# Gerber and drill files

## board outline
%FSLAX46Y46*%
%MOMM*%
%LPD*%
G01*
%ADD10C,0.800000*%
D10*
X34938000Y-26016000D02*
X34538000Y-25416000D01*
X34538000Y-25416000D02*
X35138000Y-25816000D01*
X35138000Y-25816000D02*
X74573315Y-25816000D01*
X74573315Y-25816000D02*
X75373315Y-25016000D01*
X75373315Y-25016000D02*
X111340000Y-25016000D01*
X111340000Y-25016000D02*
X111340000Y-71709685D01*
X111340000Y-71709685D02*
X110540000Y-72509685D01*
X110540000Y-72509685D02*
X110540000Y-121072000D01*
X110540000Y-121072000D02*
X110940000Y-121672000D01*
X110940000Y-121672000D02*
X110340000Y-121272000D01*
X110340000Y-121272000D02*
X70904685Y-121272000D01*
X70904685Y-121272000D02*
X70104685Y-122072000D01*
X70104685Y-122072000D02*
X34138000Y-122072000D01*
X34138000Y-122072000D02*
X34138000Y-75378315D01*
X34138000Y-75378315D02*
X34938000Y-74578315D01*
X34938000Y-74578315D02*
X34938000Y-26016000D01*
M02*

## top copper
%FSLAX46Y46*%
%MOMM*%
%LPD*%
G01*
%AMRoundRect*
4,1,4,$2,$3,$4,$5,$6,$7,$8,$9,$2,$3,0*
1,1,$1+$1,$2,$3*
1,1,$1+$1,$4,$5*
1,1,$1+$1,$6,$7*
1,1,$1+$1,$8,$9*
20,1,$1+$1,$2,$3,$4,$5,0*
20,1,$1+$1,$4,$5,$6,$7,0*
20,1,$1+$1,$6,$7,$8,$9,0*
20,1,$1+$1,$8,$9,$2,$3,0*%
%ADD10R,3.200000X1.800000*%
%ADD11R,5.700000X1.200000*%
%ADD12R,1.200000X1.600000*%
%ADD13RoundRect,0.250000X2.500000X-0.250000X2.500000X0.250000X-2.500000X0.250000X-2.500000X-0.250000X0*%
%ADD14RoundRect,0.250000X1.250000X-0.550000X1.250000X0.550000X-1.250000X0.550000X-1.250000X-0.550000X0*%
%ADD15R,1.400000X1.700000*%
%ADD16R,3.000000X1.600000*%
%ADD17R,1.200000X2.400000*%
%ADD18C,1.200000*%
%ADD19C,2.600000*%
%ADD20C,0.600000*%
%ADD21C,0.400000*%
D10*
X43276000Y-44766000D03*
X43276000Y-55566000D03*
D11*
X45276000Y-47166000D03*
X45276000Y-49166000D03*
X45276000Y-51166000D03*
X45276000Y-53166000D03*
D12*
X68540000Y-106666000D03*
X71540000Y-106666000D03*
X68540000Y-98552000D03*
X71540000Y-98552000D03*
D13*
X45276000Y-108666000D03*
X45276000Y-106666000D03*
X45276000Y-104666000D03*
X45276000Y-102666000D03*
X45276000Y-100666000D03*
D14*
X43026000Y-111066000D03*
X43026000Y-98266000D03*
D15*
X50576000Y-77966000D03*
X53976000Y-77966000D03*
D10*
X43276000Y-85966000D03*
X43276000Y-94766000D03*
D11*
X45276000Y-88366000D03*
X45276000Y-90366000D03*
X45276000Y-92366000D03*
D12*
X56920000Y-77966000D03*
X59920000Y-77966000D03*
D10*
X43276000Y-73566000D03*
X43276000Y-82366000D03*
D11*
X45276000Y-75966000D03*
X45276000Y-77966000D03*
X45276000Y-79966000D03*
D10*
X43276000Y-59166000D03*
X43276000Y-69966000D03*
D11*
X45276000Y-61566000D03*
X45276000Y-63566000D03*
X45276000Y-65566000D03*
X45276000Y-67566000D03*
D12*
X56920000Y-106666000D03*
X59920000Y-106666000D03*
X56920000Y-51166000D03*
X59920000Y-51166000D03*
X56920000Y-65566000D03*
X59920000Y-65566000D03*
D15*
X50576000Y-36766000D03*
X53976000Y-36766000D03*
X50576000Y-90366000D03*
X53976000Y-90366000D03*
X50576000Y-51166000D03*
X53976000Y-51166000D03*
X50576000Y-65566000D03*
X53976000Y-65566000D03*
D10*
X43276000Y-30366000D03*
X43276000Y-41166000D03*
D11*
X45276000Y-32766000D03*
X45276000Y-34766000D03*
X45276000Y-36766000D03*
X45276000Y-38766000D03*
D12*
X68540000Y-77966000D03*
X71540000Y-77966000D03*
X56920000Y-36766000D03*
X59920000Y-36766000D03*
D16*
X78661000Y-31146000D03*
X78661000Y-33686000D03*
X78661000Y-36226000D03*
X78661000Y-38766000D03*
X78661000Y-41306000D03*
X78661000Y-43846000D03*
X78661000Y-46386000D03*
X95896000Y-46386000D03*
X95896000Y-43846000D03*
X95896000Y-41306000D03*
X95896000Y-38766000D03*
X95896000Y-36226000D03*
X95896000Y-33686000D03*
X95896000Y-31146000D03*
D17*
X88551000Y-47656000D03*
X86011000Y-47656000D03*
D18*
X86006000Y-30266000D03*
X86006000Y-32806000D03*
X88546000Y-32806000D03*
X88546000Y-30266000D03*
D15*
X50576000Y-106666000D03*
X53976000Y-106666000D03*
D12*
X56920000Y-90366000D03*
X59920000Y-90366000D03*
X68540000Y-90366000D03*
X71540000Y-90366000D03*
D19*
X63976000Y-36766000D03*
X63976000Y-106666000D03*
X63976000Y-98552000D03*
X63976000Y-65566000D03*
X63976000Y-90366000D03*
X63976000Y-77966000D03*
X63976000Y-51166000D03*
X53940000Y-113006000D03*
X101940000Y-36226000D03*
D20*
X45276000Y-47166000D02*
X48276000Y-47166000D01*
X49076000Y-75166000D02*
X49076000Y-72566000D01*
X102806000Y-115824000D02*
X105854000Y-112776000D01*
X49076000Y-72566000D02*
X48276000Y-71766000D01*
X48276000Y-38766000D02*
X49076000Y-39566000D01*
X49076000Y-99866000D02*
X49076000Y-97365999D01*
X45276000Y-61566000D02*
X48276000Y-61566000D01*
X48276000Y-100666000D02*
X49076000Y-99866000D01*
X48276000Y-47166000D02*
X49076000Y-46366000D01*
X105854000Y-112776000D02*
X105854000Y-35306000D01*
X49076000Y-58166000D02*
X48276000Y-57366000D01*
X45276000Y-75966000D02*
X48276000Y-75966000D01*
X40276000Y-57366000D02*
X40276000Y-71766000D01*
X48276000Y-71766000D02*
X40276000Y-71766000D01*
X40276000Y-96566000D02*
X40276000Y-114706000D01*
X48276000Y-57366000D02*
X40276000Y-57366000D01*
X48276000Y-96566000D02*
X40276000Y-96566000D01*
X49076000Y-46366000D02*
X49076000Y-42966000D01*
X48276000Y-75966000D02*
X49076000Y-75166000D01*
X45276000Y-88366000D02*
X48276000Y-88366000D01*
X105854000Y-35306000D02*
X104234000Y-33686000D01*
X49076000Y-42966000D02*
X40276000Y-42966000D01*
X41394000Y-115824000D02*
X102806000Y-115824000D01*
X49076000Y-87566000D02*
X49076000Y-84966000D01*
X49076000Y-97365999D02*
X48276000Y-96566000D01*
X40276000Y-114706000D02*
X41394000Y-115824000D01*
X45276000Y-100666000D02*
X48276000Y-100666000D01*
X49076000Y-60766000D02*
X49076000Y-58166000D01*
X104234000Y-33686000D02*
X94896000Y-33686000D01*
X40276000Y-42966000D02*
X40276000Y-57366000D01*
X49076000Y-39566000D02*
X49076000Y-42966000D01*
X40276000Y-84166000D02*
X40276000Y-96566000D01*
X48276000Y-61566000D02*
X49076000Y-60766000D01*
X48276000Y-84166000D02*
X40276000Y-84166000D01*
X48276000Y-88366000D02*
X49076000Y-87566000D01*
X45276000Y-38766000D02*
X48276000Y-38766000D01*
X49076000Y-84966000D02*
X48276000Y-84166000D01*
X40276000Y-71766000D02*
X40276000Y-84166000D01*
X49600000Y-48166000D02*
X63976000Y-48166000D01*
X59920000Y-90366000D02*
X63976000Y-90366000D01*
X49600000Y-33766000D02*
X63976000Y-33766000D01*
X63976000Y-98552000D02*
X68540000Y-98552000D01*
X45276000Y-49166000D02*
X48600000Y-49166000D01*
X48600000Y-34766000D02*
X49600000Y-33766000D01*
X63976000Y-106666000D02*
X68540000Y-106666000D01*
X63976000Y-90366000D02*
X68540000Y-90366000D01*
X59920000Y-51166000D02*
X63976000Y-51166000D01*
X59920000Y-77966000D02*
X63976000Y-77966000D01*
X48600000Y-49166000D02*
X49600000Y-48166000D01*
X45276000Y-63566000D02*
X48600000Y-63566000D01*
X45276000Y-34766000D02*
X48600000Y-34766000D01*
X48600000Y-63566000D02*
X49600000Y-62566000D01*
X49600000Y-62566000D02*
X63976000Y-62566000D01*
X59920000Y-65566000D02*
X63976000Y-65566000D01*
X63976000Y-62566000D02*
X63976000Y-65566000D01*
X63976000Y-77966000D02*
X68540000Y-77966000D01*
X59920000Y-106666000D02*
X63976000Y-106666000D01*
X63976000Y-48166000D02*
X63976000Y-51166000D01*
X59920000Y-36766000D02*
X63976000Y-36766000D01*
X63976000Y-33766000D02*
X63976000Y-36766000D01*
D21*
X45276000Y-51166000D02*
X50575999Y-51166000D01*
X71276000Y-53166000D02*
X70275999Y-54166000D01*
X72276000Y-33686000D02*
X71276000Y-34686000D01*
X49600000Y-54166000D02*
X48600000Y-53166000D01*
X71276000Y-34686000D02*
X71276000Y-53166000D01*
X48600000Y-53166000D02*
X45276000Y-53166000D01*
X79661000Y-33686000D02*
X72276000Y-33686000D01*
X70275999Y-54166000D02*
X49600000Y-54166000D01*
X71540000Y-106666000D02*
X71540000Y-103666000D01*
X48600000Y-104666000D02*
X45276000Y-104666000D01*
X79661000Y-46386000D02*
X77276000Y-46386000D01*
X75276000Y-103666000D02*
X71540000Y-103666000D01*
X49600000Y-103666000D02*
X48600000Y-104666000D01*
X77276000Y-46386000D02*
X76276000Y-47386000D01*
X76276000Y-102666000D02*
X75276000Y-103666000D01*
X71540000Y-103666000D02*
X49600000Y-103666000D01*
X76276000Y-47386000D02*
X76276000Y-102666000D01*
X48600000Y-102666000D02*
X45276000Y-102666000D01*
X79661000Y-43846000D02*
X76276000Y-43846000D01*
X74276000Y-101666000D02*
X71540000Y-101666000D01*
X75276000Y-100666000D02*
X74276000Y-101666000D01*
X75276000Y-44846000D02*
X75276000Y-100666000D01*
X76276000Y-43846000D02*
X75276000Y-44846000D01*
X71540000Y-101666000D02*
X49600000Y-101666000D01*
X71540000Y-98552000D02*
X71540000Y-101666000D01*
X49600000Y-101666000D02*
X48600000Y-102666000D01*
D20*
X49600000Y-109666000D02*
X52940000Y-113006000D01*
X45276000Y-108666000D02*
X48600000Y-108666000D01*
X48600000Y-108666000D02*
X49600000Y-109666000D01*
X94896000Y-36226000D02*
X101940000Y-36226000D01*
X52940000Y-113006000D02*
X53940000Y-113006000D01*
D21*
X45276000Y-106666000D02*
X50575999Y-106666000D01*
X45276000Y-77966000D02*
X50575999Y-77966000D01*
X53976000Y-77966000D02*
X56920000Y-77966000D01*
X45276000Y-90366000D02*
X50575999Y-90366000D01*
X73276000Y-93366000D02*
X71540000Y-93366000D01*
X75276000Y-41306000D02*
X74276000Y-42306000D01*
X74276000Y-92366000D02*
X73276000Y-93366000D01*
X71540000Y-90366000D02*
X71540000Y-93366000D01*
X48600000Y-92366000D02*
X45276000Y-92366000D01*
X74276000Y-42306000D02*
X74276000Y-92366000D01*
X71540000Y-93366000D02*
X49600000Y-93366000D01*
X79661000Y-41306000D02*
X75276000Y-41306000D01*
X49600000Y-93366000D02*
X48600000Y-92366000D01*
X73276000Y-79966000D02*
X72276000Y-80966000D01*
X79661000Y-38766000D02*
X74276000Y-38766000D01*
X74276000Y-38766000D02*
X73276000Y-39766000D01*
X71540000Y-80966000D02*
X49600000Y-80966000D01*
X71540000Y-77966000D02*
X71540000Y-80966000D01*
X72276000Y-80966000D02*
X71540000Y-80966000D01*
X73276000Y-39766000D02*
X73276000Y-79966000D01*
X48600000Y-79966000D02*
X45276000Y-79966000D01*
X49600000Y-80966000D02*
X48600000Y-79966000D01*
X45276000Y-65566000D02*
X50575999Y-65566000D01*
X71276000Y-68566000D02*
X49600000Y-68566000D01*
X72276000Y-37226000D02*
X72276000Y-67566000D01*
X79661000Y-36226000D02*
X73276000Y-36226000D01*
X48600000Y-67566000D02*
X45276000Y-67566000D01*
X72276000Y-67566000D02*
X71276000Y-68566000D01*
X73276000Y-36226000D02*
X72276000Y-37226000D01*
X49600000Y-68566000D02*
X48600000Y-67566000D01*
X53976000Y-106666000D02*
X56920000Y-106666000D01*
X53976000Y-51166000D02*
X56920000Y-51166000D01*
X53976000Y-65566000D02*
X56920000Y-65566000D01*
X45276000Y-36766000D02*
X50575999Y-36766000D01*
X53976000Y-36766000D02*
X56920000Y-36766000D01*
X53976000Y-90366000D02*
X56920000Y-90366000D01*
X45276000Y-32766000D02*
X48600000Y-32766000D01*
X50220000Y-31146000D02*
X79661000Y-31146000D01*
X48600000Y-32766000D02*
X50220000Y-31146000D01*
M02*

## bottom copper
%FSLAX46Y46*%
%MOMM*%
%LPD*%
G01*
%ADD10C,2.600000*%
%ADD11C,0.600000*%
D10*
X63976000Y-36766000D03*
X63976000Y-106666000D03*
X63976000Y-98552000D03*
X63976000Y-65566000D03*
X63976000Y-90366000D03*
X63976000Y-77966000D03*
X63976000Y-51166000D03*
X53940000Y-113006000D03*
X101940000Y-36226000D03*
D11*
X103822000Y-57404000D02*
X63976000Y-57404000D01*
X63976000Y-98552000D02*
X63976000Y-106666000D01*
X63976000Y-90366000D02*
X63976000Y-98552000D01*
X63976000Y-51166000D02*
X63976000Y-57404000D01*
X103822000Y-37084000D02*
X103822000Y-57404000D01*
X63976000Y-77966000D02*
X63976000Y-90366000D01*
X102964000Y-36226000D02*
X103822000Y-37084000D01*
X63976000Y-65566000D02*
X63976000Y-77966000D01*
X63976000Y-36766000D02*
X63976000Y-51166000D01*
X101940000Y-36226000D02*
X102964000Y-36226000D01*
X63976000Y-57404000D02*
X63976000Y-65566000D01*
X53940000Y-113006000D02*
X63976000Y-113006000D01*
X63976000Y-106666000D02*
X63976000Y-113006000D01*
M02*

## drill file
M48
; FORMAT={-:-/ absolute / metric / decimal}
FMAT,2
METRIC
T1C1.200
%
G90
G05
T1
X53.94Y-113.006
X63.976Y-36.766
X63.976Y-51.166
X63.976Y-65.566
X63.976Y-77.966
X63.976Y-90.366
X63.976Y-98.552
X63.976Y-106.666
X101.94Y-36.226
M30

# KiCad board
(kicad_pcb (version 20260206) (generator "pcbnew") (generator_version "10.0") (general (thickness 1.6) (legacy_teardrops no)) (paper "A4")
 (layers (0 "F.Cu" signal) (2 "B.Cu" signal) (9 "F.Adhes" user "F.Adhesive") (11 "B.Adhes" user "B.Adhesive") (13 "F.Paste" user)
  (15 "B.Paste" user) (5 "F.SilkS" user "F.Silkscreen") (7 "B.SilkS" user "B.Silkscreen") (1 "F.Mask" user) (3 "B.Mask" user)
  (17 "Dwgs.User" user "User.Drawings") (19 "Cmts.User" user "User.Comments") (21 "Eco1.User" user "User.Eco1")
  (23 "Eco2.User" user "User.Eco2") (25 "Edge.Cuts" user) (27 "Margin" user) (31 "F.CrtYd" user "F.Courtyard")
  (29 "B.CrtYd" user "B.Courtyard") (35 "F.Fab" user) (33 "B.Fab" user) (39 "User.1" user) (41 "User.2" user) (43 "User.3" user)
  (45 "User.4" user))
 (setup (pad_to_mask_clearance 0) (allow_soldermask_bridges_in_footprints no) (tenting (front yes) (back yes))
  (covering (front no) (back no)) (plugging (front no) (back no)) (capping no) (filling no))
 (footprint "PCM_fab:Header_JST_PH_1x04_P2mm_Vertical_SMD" (layer "F.Cu") (at 45.276 48.166)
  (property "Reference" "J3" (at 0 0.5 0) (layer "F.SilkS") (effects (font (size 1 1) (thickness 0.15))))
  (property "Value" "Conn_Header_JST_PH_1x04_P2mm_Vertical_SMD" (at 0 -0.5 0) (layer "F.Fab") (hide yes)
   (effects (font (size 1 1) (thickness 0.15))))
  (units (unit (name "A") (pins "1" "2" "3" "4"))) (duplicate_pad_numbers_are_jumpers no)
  (pad "" smd rect (at -2 -3.4) (size 3.2 1.8) (layers "F.Cu" "F.Mask" "F.Paste"))
  (pad "" smd rect (at -2 7.4) (size 3.2 1.8) (layers "F.Cu" "F.Mask" "F.Paste"))
  (pad "1" smd rect (at 0 -1) (size 5.7 1.2) (layers "F.Cu" "F.Mask" "F.Paste") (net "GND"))
  (pad "2" smd rect (at 0 1) (size 5.7 1.2) (layers "F.Cu" "F.Mask" "F.Paste") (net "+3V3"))
  (pad "3" smd rect (at 0 3) (size 5.7 1.2) (layers "F.Cu" "F.Mask" "F.Paste") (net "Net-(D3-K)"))
  (pad "4" smd rect (at 0 5) (size 5.7 1.2) (layers "F.Cu" "F.Mask" "F.Paste") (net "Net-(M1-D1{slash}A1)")))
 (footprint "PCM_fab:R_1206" (layer "F.Cu") (at 70.04 106.666)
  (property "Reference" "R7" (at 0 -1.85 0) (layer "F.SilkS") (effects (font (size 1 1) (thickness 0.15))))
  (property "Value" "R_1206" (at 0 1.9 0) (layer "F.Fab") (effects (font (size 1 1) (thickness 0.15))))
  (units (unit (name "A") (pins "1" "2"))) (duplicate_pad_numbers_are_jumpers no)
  (pad "1" smd rect (at -1.5 0) (size 1.2 1.6) (layers "F.Cu" "F.Mask" "F.Paste") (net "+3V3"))
  (pad "2" smd rect (at 1.5 0) (size 1.2 1.6) (layers "F.Cu" "F.Mask" "F.Paste") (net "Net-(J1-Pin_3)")))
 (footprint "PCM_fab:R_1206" (layer "F.Cu") (at 70.04 98.552)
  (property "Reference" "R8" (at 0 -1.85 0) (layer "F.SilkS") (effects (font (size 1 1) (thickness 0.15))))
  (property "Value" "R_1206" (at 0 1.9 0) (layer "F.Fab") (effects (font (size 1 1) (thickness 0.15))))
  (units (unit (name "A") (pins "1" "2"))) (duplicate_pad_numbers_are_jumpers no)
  (pad "1" smd rect (at -1.5 0) (size 1.2 1.6) (layers "F.Cu" "F.Mask" "F.Paste") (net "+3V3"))
  (pad "2" smd rect (at 1.5 0) (size 1.2 1.6) (layers "F.Cu" "F.Mask" "F.Paste") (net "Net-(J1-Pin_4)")))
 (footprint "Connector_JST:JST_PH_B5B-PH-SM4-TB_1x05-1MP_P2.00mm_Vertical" (layer "F.Cu") (at 44.776 104.666 90)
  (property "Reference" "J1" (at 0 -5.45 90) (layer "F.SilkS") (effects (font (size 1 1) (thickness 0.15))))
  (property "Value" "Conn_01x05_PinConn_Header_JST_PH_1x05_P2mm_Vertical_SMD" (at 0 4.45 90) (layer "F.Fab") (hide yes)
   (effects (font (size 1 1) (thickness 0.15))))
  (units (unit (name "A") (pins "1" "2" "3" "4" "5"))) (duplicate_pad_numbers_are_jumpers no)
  (pad "1" smd roundrect (at -4 0.5 90) (size 1 5.5) (layers "F.Cu" "F.Mask" "F.Paste") (roundrect_rratio 0.25) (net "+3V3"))
  (pad "2" smd roundrect (at -2 0.5 90) (size 1 5.5) (layers "F.Cu" "F.Mask" "F.Paste") (roundrect_rratio 0.25) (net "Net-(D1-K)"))
  (pad "3" smd roundrect (at 0 0.5 90) (size 1 5.5) (layers "F.Cu" "F.Mask" "F.Paste") (roundrect_rratio 0.25) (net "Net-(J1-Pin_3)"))
  (pad "4" smd roundrect (at 2 0.5 90) (size 1 5.5) (layers "F.Cu" "F.Mask" "F.Paste") (roundrect_rratio 0.25) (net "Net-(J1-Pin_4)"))
  (pad "5" smd roundrect (at 4 0.5 90) (size 1 5.5) (layers "F.Cu" "F.Mask" "F.Paste") (roundrect_rratio 0.25) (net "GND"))
  (pad "MP" smd roundrect (at -6.4 -1.75 90) (size 1.6 3) (layers "F.Cu" "F.Mask" "F.Paste") (roundrect_rratio 0.15625))
  (pad "MP" smd roundrect (at 6.4 -1.75 90) (size 1.6 3) (layers "F.Cu" "F.Mask" "F.Paste") (roundrect_rratio 0.15625)))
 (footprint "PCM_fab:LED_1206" (layer "F.Cu") (at 52.276 77.966)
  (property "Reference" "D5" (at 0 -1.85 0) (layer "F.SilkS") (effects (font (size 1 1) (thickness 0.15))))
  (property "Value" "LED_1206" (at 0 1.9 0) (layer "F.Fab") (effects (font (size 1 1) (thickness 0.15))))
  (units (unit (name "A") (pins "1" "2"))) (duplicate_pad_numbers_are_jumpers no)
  (pad "1" smd rect (at -1.7 0) (size 1.4 1.7) (layers "F.Cu" "F.Mask" "F.Paste") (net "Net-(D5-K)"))
  (pad "2" smd rect (at 1.7 0) (size 1.4 1.7) (layers "F.Cu" "F.Mask" "F.Paste") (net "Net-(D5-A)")))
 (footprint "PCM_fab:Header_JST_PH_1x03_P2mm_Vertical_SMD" (layer "F.Cu") (at 45.276 89.366)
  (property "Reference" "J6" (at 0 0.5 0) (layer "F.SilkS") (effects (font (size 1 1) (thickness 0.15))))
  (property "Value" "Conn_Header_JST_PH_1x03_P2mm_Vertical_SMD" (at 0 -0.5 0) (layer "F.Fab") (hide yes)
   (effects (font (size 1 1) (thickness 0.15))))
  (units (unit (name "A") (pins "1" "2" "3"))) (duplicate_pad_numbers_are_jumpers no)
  (pad "" smd rect (at -2 -3.4) (size 3.2 1.8) (layers "F.Cu" "F.Mask" "F.Paste"))
  (pad "" smd rect (at -2 5.4) (size 3.2 1.8) (layers "F.Cu" "F.Mask" "F.Paste"))
  (pad "1" smd rect (at 0 -1) (size 5.7 1.2) (layers "F.Cu" "F.Mask" "F.Paste") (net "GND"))
  (pad "2" smd rect (at 0 1) (size 5.7 1.2) (layers "F.Cu" "F.Mask" "F.Paste") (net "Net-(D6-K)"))
  (pad "3" smd rect (at 0 3) (size 5.7 1.2) (layers "F.Cu" "F.Mask" "F.Paste") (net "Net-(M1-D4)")))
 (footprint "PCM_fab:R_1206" (layer "F.Cu") (at 58.42 77.966)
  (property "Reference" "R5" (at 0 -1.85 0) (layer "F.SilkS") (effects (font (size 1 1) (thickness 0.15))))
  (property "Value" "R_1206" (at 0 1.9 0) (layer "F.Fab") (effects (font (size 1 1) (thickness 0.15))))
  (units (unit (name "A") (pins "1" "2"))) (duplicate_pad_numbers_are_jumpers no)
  (pad "1" smd rect (at -1.5 0) (size 1.2 1.6) (layers "F.Cu" "F.Mask" "F.Paste") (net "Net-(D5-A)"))
  (pad "2" smd rect (at 1.5 0) (size 1.2 1.6) (layers "F.Cu" "F.Mask" "F.Paste") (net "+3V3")))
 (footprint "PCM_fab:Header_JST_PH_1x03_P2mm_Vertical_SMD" (layer "F.Cu") (at 45.276 76.966)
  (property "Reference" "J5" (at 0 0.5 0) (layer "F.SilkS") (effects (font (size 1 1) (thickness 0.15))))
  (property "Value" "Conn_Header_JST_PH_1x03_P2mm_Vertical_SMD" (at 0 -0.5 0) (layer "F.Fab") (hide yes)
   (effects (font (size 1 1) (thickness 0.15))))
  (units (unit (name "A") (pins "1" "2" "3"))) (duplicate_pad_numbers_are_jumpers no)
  (pad "" smd rect (at -2 -3.4) (size 3.2 1.8) (layers "F.Cu" "F.Mask" "F.Paste"))
  (pad "" smd rect (at -2 5.4) (size 3.2 1.8) (layers "F.Cu" "F.Mask" "F.Paste"))
  (pad "1" smd rect (at 0 -1) (size 5.7 1.2) (layers "F.Cu" "F.Mask" "F.Paste") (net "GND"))
  (pad "2" smd rect (at 0 1) (size 5.7 1.2) (layers "F.Cu" "F.Mask" "F.Paste") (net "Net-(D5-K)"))
  (pad "3" smd rect (at 0 3) (size 5.7 1.2) (layers "F.Cu" "F.Mask" "F.Paste") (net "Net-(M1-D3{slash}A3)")))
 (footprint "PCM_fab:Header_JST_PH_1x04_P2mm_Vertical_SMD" (layer "F.Cu") (at 45.276 62.566)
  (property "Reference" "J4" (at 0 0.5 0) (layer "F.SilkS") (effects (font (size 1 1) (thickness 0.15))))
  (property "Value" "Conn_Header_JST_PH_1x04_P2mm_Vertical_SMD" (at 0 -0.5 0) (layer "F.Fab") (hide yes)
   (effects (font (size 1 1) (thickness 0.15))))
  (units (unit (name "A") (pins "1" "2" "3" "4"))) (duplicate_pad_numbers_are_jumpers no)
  (pad "" smd rect (at -2 -3.4) (size 3.2 1.8) (layers "F.Cu" "F.Mask" "F.Paste"))
  (pad "" smd rect (at -2 7.4) (size 3.2 1.8) (layers "F.Cu" "F.Mask" "F.Paste"))
  (pad "1" smd rect (at 0 -1) (size 5.7 1.2) (layers "F.Cu" "F.Mask" "F.Paste") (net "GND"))
  (pad "2" smd rect (at 0 1) (size 5.7 1.2) (layers "F.Cu" "F.Mask" "F.Paste") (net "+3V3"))
  (pad "3" smd rect (at 0 3) (size 5.7 1.2) (layers "F.Cu" "F.Mask" "F.Paste") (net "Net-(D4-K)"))
  (pad "4" smd rect (at 0 5) (size 5.7 1.2) (layers "F.Cu" "F.Mask" "F.Paste") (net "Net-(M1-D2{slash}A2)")))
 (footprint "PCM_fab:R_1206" (layer "F.Cu") (at 58.42 106.666)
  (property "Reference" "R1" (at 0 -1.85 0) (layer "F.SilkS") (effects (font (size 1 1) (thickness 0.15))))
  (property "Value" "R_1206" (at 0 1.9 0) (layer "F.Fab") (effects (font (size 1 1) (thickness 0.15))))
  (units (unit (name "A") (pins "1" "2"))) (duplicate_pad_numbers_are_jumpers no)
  (pad "1" smd rect (at -1.5 0) (size 1.2 1.6) (layers "F.Cu" "F.Mask" "F.Paste") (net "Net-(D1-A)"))
  (pad "2" smd rect (at 1.5 0) (size 1.2 1.6) (layers "F.Cu" "F.Mask" "F.Paste") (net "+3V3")))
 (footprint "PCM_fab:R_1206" (layer "F.Cu") (at 58.42 51.166)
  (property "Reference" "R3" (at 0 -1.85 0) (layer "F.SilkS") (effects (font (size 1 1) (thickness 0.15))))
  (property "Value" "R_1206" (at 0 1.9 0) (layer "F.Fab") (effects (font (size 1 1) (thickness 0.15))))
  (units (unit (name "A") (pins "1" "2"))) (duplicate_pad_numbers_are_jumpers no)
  (pad "1" smd rect (at -1.5 0) (size 1.2 1.6) (layers "F.Cu" "F.Mask" "F.Paste") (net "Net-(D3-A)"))
  (pad "2" smd rect (at 1.5 0) (size 1.2 1.6) (layers "F.Cu" "F.Mask" "F.Paste") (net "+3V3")))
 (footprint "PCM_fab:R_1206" (layer "F.Cu") (at 58.42 65.566)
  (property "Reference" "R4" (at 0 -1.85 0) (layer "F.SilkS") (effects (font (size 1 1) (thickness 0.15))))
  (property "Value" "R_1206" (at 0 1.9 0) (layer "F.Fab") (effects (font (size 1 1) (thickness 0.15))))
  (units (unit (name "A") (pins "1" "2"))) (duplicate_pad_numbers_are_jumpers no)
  (pad "1" smd rect (at -1.5 0) (size 1.2 1.6) (layers "F.Cu" "F.Mask" "F.Paste") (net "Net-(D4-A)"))
  (pad "2" smd rect (at 1.5 0) (size 1.2 1.6) (layers "F.Cu" "F.Mask" "F.Paste") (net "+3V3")))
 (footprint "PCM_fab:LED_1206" (layer "F.Cu") (at 52.276 36.766)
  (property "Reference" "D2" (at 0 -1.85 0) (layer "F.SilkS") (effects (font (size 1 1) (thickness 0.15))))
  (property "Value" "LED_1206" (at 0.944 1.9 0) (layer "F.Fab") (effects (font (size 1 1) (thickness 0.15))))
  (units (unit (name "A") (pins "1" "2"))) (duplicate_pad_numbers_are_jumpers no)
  (pad "1" smd rect (at -1.7 0) (size 1.4 1.7) (layers "F.Cu" "F.Mask" "F.Paste") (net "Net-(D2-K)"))
  (pad "2" smd rect (at 1.7 0) (size 1.4 1.7) (layers "F.Cu" "F.Mask" "F.Paste") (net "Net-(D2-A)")))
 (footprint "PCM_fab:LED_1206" (layer "F.Cu") (at 52.276 90.366)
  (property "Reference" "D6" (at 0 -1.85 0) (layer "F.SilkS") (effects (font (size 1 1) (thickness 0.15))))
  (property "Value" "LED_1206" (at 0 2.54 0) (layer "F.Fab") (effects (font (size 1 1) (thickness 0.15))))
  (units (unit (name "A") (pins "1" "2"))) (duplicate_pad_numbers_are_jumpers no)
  (pad "1" smd rect (at -1.7 0) (size 1.4 1.7) (layers "F.Cu" "F.Mask" "F.Paste") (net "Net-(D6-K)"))
  (pad "2" smd rect (at 1.7 0) (size 1.4 1.7) (layers "F.Cu" "F.Mask" "F.Paste") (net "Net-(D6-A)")))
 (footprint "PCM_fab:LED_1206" (layer "F.Cu") (at 52.276 51.166)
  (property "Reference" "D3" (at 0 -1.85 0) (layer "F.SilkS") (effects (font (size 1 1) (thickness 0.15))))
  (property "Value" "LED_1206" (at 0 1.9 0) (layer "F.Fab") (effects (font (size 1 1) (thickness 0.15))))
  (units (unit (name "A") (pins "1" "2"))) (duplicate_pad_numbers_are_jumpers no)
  (pad "1" smd rect (at -1.7 0) (size 1.4 1.7) (layers "F.Cu" "F.Mask" "F.Paste") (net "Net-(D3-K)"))
  (pad "2" smd rect (at 1.7 0) (size 1.4 1.7) (layers "F.Cu" "F.Mask" "F.Paste") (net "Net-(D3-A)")))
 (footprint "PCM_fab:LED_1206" (layer "F.Cu") (at 52.276 65.566)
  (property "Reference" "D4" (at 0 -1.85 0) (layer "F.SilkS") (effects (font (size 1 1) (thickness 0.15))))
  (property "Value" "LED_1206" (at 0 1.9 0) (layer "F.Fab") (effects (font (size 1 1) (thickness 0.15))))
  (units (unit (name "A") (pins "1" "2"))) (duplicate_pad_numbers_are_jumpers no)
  (pad "1" smd rect (at -1.7 0) (size 1.4 1.7) (layers "F.Cu" "F.Mask" "F.Paste") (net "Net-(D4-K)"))
  (pad "2" smd rect (at 1.7 0) (size 1.4 1.7) (layers "F.Cu" "F.Mask" "F.Paste") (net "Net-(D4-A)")))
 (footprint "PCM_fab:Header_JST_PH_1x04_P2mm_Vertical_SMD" (layer "F.Cu") (at 45.276 33.766)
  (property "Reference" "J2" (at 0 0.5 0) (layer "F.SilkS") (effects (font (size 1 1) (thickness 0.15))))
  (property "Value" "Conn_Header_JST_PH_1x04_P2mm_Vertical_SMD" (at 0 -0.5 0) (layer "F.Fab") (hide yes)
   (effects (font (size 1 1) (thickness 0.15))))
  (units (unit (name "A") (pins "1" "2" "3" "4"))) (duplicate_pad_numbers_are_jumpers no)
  (pad "" smd rect (at -2 -3.4) (size 3.2 1.8) (layers "F.Cu" "F.Mask" "F.Paste"))
  (pad "" smd rect (at -2 7.4) (size 3.2 1.8) (layers "F.Cu" "F.Mask" "F.Paste"))
  (pad "1" smd rect (at 0 -1) (size 5.7 1.2) (layers "F.Cu" "F.Mask" "F.Paste") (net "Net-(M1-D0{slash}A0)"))
  (pad "2" smd rect (at 0 1) (size 5.7 1.2) (layers "F.Cu" "F.Mask" "F.Paste") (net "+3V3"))
  (pad "3" smd rect (at 0 3) (size 5.7 1.2) (layers "F.Cu" "F.Mask" "F.Paste") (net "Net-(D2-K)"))
  (pad "4" smd rect (at 0 5) (size 5.7 1.2) (layers "F.Cu" "F.Mask" "F.Paste") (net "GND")))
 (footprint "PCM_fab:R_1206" (layer "F.Cu") (at 70.04 77.966)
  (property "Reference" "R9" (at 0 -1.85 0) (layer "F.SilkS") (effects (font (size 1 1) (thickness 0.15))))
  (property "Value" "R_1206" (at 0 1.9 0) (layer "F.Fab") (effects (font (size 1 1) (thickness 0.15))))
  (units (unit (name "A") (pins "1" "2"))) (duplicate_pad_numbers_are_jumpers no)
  (pad "1" smd rect (at -1.5 0) (size 1.2 1.6) (layers "F.Cu" "F.Mask" "F.Paste") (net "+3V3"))
  (pad "2" smd rect (at 1.5 0) (size 1.2 1.6) (layers "F.Cu" "F.Mask" "F.Paste") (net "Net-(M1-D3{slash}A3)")))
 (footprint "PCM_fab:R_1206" (layer "F.Cu") (at 58.42 36.766)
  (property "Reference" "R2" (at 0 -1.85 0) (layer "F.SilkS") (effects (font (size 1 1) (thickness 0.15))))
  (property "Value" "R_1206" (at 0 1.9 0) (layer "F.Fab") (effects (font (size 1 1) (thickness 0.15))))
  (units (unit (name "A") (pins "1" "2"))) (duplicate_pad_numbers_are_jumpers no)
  (pad "1" smd rect (at -1.5 0) (size 1.2 1.6) (layers "F.Cu" "F.Mask" "F.Paste") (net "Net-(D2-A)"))
  (pad "2" smd rect (at 1.5 0) (size 1.2 1.6) (layers "F.Cu" "F.Mask" "F.Paste") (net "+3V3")))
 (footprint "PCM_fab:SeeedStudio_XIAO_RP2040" (layer "F.Cu") (at 87.276 38.766)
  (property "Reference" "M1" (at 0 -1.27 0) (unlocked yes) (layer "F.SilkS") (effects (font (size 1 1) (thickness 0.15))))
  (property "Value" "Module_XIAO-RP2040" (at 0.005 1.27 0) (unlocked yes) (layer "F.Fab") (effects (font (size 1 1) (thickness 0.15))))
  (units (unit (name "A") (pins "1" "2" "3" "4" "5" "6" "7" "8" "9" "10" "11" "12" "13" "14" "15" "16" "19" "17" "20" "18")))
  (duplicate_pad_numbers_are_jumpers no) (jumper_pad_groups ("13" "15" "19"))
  (pad "1" smd rect (at -7.615 -7.62) (size 3 1.6) (drill (offset -1 0)) (layers "F.Cu" "F.Mask" "F.Paste") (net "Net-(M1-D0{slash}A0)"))
  (pad "2" smd rect (at -7.615 -5.08) (size 3 1.6) (drill (offset -1 0)) (layers "F.Cu" "F.Mask" "F.Paste") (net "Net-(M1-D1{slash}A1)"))
  (pad "3" smd rect (at -7.615 -2.54) (size 3 1.6) (drill (offset -1 0)) (layers "F.Cu" "F.Mask" "F.Paste") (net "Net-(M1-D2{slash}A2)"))
  (pad "4" smd rect (at -7.615 0) (size 3 1.6) (drill (offset -1 0)) (layers "F.Cu" "F.Mask" "F.Paste") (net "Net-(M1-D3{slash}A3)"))
  (pad "5" smd rect (at -7.615 2.54) (size 3 1.6) (drill (offset -1 0)) (layers "F.Cu" "F.Mask" "F.Paste") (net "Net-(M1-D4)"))
  (pad "6" smd rect (at -7.615 5.08) (size 3 1.6) (drill (offset -1 0)) (layers "F.Cu" "F.Mask" "F.Paste") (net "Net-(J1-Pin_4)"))
  (pad "7" smd rect (at -7.615 7.62) (size 3 1.6) (drill (offset -1 0)) (layers "F.Cu" "F.Mask" "F.Paste") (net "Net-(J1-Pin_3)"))
  (pad "8" smd rect (at 7.62 7.62) (size 3 1.6) (drill (offset 1 0)) (layers "F.Cu" "F.Mask" "F.Paste") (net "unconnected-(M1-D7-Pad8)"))
  (pad "9" smd rect (at 7.62 5.08) (size 3 1.6) (drill (offset 1 0)) (layers "F.Cu" "F.Mask" "F.Paste") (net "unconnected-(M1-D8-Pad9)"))
  (pad "10" smd rect (at 7.62 2.54) (size 3 1.6) (drill (offset 1 0)) (layers "F.Cu" "F.Mask" "F.Paste") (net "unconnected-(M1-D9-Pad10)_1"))
  (pad "11" smd rect (at 7.62 0) (size 3 1.6) (drill (offset 1 0)) (layers "F.Cu" "F.Mask" "F.Paste") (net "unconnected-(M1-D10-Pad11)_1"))
  (pad "12" smd rect (at 7.62 -2.54) (size 3 1.6) (drill (offset 1 0)) (layers "F.Cu" "F.Mask" "F.Paste") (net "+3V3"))
  (pad "13" smd rect (at 7.62 -5.08) (size 3 1.6) (drill (offset 1 0)) (layers "F.Cu" "F.Mask" "F.Paste") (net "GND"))
  (pad "14" smd rect (at 7.62 -7.62) (size 3 1.6) (drill (offset 1 0)) (layers "F.Cu" "F.Mask" "F.Paste") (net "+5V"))
  (pad "15" smd rect (at 1.275 8.89 270) (size 2.4 1.2) (layers "F.Cu" "F.Mask" "F.Paste") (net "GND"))
  (pad "16" smd rect (at -1.265 8.89 270) (size 2.4 1.2) (layers "F.Cu" "F.Mask" "F.Paste") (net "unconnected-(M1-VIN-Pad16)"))
  (pad "17" smd circle (at -1.27 -8.5) (size 1.2 1.2) (layers "F.Cu" "F.Mask" "F.Paste") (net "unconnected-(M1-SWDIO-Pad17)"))
  (pad "18" smd circle (at -1.27 -5.96) (size 1.2 1.2) (layers "F.Cu" "F.Mask" "F.Paste") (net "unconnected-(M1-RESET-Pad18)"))
  (pad "19" smd circle (at 1.27 -5.96) (size 1.2 1.2) (layers "F.Cu" "F.Mask" "F.Paste") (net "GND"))
  (pad "20" smd circle (at 1.27 -8.5) (size 1.2 1.2) (layers "F.Cu" "F.Mask" "F.Paste") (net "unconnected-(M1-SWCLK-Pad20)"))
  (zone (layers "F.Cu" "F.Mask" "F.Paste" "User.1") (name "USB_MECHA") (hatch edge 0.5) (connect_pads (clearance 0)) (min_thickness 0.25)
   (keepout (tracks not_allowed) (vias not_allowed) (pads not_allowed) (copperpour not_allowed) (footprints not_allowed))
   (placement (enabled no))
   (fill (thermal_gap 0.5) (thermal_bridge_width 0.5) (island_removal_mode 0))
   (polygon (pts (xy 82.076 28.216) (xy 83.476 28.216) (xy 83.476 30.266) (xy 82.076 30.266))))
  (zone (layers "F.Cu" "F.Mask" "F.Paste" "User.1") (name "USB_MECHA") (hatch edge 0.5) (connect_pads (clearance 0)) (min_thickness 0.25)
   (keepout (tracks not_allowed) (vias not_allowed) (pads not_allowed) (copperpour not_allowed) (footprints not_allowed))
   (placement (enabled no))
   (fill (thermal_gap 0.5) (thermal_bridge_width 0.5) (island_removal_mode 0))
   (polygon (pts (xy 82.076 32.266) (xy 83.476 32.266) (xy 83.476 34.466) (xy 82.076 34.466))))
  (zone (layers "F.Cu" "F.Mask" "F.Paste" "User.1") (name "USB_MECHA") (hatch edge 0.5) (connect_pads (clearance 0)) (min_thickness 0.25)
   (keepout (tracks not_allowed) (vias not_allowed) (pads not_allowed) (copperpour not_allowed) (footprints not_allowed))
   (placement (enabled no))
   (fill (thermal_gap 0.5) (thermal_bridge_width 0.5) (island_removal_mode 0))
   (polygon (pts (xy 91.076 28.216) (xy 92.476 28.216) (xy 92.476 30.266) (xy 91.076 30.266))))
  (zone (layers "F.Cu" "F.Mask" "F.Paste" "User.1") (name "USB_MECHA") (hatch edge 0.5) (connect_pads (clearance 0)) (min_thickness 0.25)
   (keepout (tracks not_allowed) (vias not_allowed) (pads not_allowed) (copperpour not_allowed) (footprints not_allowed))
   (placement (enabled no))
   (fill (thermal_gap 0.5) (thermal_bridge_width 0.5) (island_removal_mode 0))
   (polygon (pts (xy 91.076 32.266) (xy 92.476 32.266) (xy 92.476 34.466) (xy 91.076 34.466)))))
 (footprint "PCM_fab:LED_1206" (layer "F.Cu") (at 52.276 106.666)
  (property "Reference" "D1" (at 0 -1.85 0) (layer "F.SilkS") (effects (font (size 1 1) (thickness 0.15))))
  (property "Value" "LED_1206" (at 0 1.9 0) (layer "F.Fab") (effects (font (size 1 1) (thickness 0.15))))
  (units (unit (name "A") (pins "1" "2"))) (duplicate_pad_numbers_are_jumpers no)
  (pad "1" smd rect (at -1.7 0) (size 1.4 1.7) (layers "F.Cu" "F.Mask" "F.Paste") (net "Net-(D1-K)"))
  (pad "2" smd rect (at 1.7 0) (size 1.4 1.7) (layers "F.Cu" "F.Mask" "F.Paste") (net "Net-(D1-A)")))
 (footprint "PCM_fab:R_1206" (layer "F.Cu") (at 58.42 90.366)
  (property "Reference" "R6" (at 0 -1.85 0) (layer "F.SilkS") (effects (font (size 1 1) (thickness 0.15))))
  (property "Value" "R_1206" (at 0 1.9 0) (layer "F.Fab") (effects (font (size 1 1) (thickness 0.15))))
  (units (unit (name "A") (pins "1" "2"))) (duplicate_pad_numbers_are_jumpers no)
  (pad "1" smd rect (at -1.5 0) (size 1.2 1.6) (layers "F.Cu" "F.Mask" "F.Paste") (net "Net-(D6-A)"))
  (pad "2" smd rect (at 1.5 0) (size 1.2 1.6) (layers "F.Cu" "F.Mask" "F.Paste") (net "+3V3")))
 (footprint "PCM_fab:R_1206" (layer "F.Cu") (at 70.04 90.366)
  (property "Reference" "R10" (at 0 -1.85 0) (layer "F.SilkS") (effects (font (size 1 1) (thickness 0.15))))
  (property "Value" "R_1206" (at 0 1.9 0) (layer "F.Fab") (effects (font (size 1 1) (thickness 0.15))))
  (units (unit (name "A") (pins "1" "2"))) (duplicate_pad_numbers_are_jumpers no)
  (pad "1" smd rect (at -1.5 0) (size 1.2 1.6) (layers "F.Cu" "F.Mask" "F.Paste") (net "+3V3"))
  (pad "2" smd rect (at 1.5 0) (size 1.2 1.6) (layers "F.Cu" "F.Mask" "F.Paste") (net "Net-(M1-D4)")))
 (gr_line (start 34.938 26.016) (end 34.538 25.416) (stroke (width 0.8) (type solid)) (layer "Edge.Cuts"))
 (gr_line (start 34.538 25.416) (end 35.138 25.816) (stroke (width 0.8) (type solid)) (layer "Edge.Cuts"))
 (gr_line (start 35.138 25.816) (end 74.573315 25.816) (stroke (width 0.8) (type solid)) (layer "Edge.Cuts"))
 (gr_line (start 74.573315 25.816) (end 75.373315 25.016) (stroke (width 0.8) (type solid)) (layer "Edge.Cuts"))
 (gr_line (start 75.373315 25.016) (end 111.34 25.016) (stroke (width 0.8) (type solid)) (layer "Edge.Cuts"))
 (gr_line (start 111.34 25.016) (end 111.34 71.709685) (stroke (width 0.8) (type solid)) (layer "Edge.Cuts"))
 (gr_line (start 111.34 71.709685) (end 110.54 72.509685) (stroke (width 0.8) (type solid)) (layer "Edge.Cuts"))
 (gr_line (start 110.54 72.509685) (end 110.54 121.072) (stroke (width 0.8) (type solid)) (layer "Edge.Cuts"))
 (gr_line (start 110.54 121.072) (end 110.94 121.672) (stroke (width 0.8) (type solid)) (layer "Edge.Cuts"))
 (gr_line (start 110.94 121.672) (end 110.34 121.272) (stroke (width 0.8) (type solid)) (layer "Edge.Cuts"))
 (gr_line (start 110.34 121.272) (end 70.904685 121.272) (stroke (width 0.8) (type solid)) (layer "Edge.Cuts"))
 (gr_line (start 70.904685 121.272) (end 70.104685 122.072) (stroke (width 0.8) (type solid)) (layer "Edge.Cuts"))
 (gr_line (start 70.104685 122.072) (end 34.138 122.072) (stroke (width 0.8) (type solid)) (layer "Edge.Cuts"))
 (gr_line (start 34.138 122.072) (end 34.138 75.378315) (stroke (width 0.8) (type solid)) (layer "Edge.Cuts"))
 (gr_line (start 34.138 75.378315) (end 34.938 74.578315) (stroke (width 0.8) (type solid)) (layer "Edge.Cuts"))
 (gr_line (start 34.938 74.578315) (end 34.938 26.016) (stroke (width 0.8) (type solid)) (layer "Edge.Cuts"))
 (segment (start 45.276 47.166) (end 48.276 47.166) (width 0.6) (layer "F.Cu") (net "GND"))
 (segment (start 49.076 75.166) (end 49.076 72.566) (width 0.6) (layer "F.Cu") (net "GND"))
 (segment (start 102.806 115.824) (end 105.854 112.776) (width 0.6) (layer "F.Cu") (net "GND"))
 (segment (start 49.076 72.566) (end 48.276 71.766) (width 0.6) (layer "F.Cu") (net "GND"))
 (segment (start 48.276 38.766) (end 49.076 39.566) (width 0.6) (layer "F.Cu") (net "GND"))
 (segment (start 49.076 99.866) (end 49.076 97.365999) (width 0.6) (layer "F.Cu") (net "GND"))
 (segment (start 45.276 61.566) (end 48.276 61.566) (width 0.6) (layer "F.Cu") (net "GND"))
 (segment (start 48.276 100.666) (end 49.076 99.866) (width 0.6) (layer "F.Cu") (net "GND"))
 (segment (start 48.276 47.166) (end 49.076 46.366) (width 0.6) (layer "F.Cu") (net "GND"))
 (segment (start 105.854 112.776) (end 105.854 35.306) (width 0.6) (layer "F.Cu") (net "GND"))
 (segment (start 49.076 58.166) (end 48.276 57.366) (width 0.6) (layer "F.Cu") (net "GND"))
 (segment (start 45.276 75.966) (end 48.276 75.966) (width 0.6) (layer "F.Cu") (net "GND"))
 (segment (start 40.276 57.366) (end 40.276 71.766) (width 0.6) (layer "F.Cu") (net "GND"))
 (segment (start 48.276 71.766) (end 40.276 71.766) (width 0.6) (layer "F.Cu") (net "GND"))
 (segment (start 40.276 96.566) (end 40.276 114.706) (width 0.6) (layer "F.Cu") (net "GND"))
 (segment (start 48.276 57.366) (end 40.276 57.366) (width 0.6) (layer "F.Cu") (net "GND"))
 (segment (start 48.276 96.566) (end 40.276 96.566) (width 0.6) (layer "F.Cu") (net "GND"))
 (segment (start 49.076 46.366) (end 49.076 42.966) (width 0.6) (layer "F.Cu") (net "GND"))
 (segment (start 48.276 75.966) (end 49.076 75.166) (width 0.6) (layer "F.Cu") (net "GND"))
 (segment (start 45.276 88.366) (end 48.276 88.366) (width 0.6) (layer "F.Cu") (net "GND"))
 (segment (start 105.854 35.306) (end 104.234 33.686) (width 0.6) (layer "F.Cu") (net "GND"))
 (segment (start 49.076 42.966) (end 40.276 42.966) (width 0.6) (layer "F.Cu") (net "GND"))
 (segment (start 41.394 115.824) (end 102.806 115.824) (width 0.6) (layer "F.Cu") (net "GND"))
 (segment (start 49.076 87.566) (end 49.076 84.966) (width 0.6) (layer "F.Cu") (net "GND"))
 (segment (start 49.076 97.365999) (end 48.276 96.566) (width 0.6) (layer "F.Cu") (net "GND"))
 (segment (start 40.276 114.706) (end 41.394 115.824) (width 0.6) (layer "F.Cu") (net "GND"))
 (segment (start 45.276 100.666) (end 48.276 100.666) (width 0.6) (layer "F.Cu") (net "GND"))
 (segment (start 49.076 60.766) (end 49.076 58.166) (width 0.6) (layer "F.Cu") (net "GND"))
 (segment (start 104.234 33.686) (end 94.896 33.686) (width 0.6) (layer "F.Cu") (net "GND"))
 (segment (start 40.276 42.966) (end 40.276 57.366) (width 0.6) (layer "F.Cu") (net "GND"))
 (segment (start 49.076 39.566) (end 49.076 42.966) (width 0.6) (layer "F.Cu") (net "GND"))
 (segment (start 40.276 84.166) (end 40.276 96.566) (width 0.6) (layer "F.Cu") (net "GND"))
 (segment (start 48.276 61.566) (end 49.076 60.766) (width 0.6) (layer "F.Cu") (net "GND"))
 (segment (start 48.276 84.166) (end 40.276 84.166) (width 0.6) (layer "F.Cu") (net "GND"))
 (segment (start 48.276 88.366) (end 49.076 87.566) (width 0.6) (layer "F.Cu") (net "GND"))
 (segment (start 45.276 38.766) (end 48.276 38.766) (width 0.6) (layer "F.Cu") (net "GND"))
 (segment (start 49.076 84.966) (end 48.276 84.166) (width 0.6) (layer "F.Cu") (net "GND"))
 (segment (start 40.276 71.766) (end 40.276 84.166) (width 0.6) (layer "F.Cu") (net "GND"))
 (segment (start 49.6 48.166) (end 63.976 48.166) (width 0.6) (layer "F.Cu") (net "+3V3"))
 (segment (start 59.92 90.366) (end 63.976 90.366) (width 0.6) (layer "F.Cu") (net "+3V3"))
 (segment (start 49.6 33.766) (end 63.976 33.766) (width 0.6) (layer "F.Cu") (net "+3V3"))
 (segment (start 63.976 98.552) (end 68.54 98.552) (width 0.6) (layer "F.Cu") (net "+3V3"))
 (segment (start 45.276 49.166) (end 48.6 49.166) (width 0.6) (layer "F.Cu") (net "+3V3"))
 (segment (start 48.6 34.766) (end 49.6 33.766) (width 0.6) (layer "F.Cu") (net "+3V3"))
 (segment (start 63.976 106.666) (end 68.54 106.666) (width 0.6) (layer "F.Cu") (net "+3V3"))
 (segment (start 63.976 90.366) (end 68.54 90.366) (width 0.6) (layer "F.Cu") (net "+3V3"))
 (segment (start 59.92 51.166) (end 63.976 51.166) (width 0.6) (layer "F.Cu") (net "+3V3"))
 (segment (start 59.92 77.966) (end 63.976 77.966) (width 0.6) (layer "F.Cu") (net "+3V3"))
 (segment (start 48.6 49.166) (end 49.6 48.166) (width 0.6) (layer "F.Cu") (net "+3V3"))
 (segment (start 45.276 63.566) (end 48.6 63.566) (width 0.6) (layer "F.Cu") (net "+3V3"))
 (segment (start 45.276 34.766) (end 48.6 34.766) (width 0.6) (layer "F.Cu") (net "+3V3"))
 (segment (start 48.6 63.566) (end 49.6 62.566) (width 0.6) (layer "F.Cu") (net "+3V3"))
 (segment (start 49.6 62.566) (end 63.976 62.566) (width 0.6) (layer "F.Cu") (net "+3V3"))
 (segment (start 59.92 65.566) (end 63.976 65.566) (width 0.6) (layer "F.Cu") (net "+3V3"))
 (segment (start 63.976 62.566) (end 63.976 65.566) (width 0.6) (layer "F.Cu") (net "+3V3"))
 (segment (start 63.976 77.966) (end 68.54 77.966) (width 0.6) (layer "F.Cu") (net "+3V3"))
 (segment (start 59.92 106.666) (end 63.976 106.666) (width 0.6) (layer "F.Cu") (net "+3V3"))
 (segment (start 63.976 48.166) (end 63.976 51.166) (width 0.6) (layer "F.Cu") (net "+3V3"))
 (segment (start 59.92 36.766) (end 63.976 36.766) (width 0.6) (layer "F.Cu") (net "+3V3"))
 (segment (start 63.976 33.766) (end 63.976 36.766) (width 0.6) (layer "F.Cu") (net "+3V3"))
 (via (at 63.976 36.766) (size 2.6) (drill 1.2) (layers "F.Cu" "B.Cu") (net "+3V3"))
 (via (at 63.976 106.666) (size 2.6) (drill 1.2) (layers "F.Cu" "B.Cu") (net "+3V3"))
 (via (at 63.976 98.552) (size 2.6) (drill 1.2) (layers "F.Cu" "B.Cu") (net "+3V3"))
 (via (at 63.976 65.566) (size 2.6) (drill 1.2) (layers "F.Cu" "B.Cu") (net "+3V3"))
 (via (at 63.976 90.366) (size 2.6) (drill 1.2) (layers "F.Cu" "B.Cu") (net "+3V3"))
 (via (at 63.976 77.966) (size 2.6) (drill 1.2) (layers "F.Cu" "B.Cu") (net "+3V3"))
 (via (at 63.976 51.166) (size 2.6) (drill 1.2) (layers "F.Cu" "B.Cu") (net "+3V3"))
 (segment (start 103.822 57.404) (end 63.976 57.404) (width 0.6) (layer "B.Cu") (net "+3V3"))
 (segment (start 63.976 98.552) (end 63.976 106.666) (width 0.6) (layer "B.Cu") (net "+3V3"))
 (segment (start 63.976 90.366) (end 63.976 98.552) (width 0.6) (layer "B.Cu") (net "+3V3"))
 (segment (start 63.976 51.166) (end 63.976 57.404) (width 0.6) (layer "B.Cu") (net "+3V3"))
 (segment (start 103.822 37.084) (end 103.822 57.404) (width 0.6) (layer "B.Cu") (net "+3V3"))
 (segment (start 63.976 77.966) (end 63.976 90.366) (width 0.6) (layer "B.Cu") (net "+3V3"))
 (segment (start 102.964 36.226) (end 103.822 37.084) (width 0.6) (layer "B.Cu") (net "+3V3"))
 (segment (start 63.976 65.566) (end 63.976 77.966) (width 0.6) (layer "B.Cu") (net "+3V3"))
 (segment (start 63.976 36.766) (end 63.976 51.166) (width 0.6) (layer "B.Cu") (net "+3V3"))
 (segment (start 101.94 36.226) (end 102.964 36.226) (width 0.6) (layer "B.Cu") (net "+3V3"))
 (segment (start 63.976 57.404) (end 63.976 65.566) (width 0.6) (layer "B.Cu") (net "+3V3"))
 (segment (start 45.276 51.166) (end 50.575999 51.166) (width 0.4) (layer "F.Cu") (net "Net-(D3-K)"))
 (segment (start 71.276 53.166) (end 70.275999 54.166) (width 0.4) (layer "F.Cu") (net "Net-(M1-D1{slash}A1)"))
 (segment (start 72.276 33.686) (end 71.276 34.686) (width 0.4) (layer "F.Cu") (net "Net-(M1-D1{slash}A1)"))
 (segment (start 49.6 54.166) (end 48.6 53.166) (width 0.4) (layer "F.Cu") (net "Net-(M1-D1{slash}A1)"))
 (segment (start 71.276 34.686) (end 71.276 53.166) (width 0.4) (layer "F.Cu") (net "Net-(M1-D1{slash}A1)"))
 (segment (start 48.6 53.166) (end 45.276 53.166) (width 0.4) (layer "F.Cu") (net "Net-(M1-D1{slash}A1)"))
 (segment (start 79.661 33.686) (end 72.276 33.686) (width 0.4) (layer "F.Cu") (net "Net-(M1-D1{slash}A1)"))
 (segment (start 70.275999 54.166) (end 49.6 54.166) (width 0.4) (layer "F.Cu") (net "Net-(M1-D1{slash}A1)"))
 (segment (start 71.54 106.666) (end 71.54 103.666) (width 0.4) (layer "F.Cu") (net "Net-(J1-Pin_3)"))
 (segment (start 48.6 104.666) (end 45.276 104.666) (width 0.4) (layer "F.Cu") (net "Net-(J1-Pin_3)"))
 (segment (start 79.661 46.386) (end 77.276 46.386) (width 0.4) (layer "F.Cu") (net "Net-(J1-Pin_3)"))
 (segment (start 75.276 103.666) (end 71.54 103.666) (width 0.4) (layer "F.Cu") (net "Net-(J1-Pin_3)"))
 (segment (start 49.6 103.666) (end 48.6 104.666) (width 0.4) (layer "F.Cu") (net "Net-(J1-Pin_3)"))
 (segment (start 77.276 46.386) (end 76.276 47.386) (width 0.4) (layer "F.Cu") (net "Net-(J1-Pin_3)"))
 (segment (start 76.276 102.666) (end 75.276 103.666) (width 0.4) (layer "F.Cu") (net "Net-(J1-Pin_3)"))
 (segment (start 71.54 103.666) (end 49.6 103.666) (width 0.4) (layer "F.Cu") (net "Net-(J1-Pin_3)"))
 (segment (start 76.276 47.386) (end 76.276 102.666) (width 0.4) (layer "F.Cu") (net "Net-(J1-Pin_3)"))
 (segment (start 48.6 102.666) (end 45.276 102.666) (width 0.4) (layer "F.Cu") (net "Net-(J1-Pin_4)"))
 (segment (start 79.661 43.846) (end 76.276 43.846) (width 0.4) (layer "F.Cu") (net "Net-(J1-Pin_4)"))
 (segment (start 74.276 101.666) (end 71.54 101.666) (width 0.4) (layer "F.Cu") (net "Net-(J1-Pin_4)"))
 (segment (start 75.276 100.666) (end 74.276 101.666) (width 0.4) (layer "F.Cu") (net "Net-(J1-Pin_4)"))
 (segment (start 75.276 44.846) (end 75.276 100.666) (width 0.4) (layer "F.Cu") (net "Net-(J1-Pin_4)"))
 (segment (start 76.276 43.846) (end 75.276 44.846) (width 0.4) (layer "F.Cu") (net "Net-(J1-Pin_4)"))
 (segment (start 71.54 101.666) (end 49.6 101.666) (width 0.4) (layer "F.Cu") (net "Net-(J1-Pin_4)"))
 (segment (start 71.54 98.552) (end 71.54 101.666) (width 0.4) (layer "F.Cu") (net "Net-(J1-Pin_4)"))
 (segment (start 49.6 101.666) (end 48.6 102.666) (width 0.4) (layer "F.Cu") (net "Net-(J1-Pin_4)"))
 (segment (start 49.6 109.666) (end 52.94 113.006) (width 0.6) (layer "F.Cu") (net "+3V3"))
 (segment (start 45.276 108.666) (end 48.6 108.666) (width 0.6) (layer "F.Cu") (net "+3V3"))
 (segment (start 48.6 108.666) (end 49.6 109.666) (width 0.6) (layer "F.Cu") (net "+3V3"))
 (via (at 53.94 113.006) (size 2.6) (drill 1.2) (layers "F.Cu" "B.Cu") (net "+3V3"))
 (segment (start 94.896 36.226) (end 101.94 36.226) (width 0.6) (layer "F.Cu") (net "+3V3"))
 (via (at 101.94 36.226) (size 2.6) (drill 1.2) (layers "F.Cu" "B.Cu") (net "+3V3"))
 (segment (start 52.94 113.006) (end 53.94 113.006) (width 0.6) (layer "F.Cu") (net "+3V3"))
 (segment (start 53.94 113.006) (end 63.976 113.006) (width 0.6) (layer "B.Cu") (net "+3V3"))
 (segment (start 63.976 106.666) (end 63.976 113.006) (width 0.6) (layer "B.Cu") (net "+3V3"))
 (segment (start 45.276 106.666) (end 50.575999 106.666) (width 0.4) (layer "F.Cu") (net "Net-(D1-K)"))
 (segment (start 45.276 77.966) (end 50.575999 77.966) (width 0.4) (layer "F.Cu") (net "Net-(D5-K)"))
 (segment (start 53.976 77.966) (end 56.92 77.966) (width 0.4) (layer "F.Cu") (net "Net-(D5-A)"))
 (segment (start 45.276 90.366) (end 50.575999 90.366) (width 0.4) (layer "F.Cu") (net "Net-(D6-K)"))
 (segment (start 73.276 93.366) (end 71.54 93.366) (width 0.4) (layer "F.Cu") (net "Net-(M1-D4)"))
 (segment (start 75.276 41.306) (end 74.276 42.306) (width 0.4) (layer "F.Cu") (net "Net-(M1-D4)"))
 (segment (start 74.276 92.366) (end 73.276 93.366) (width 0.4) (layer "F.Cu") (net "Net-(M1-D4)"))
 (segment (start 71.54 90.366) (end 71.54 93.366) (width 0.4) (layer "F.Cu") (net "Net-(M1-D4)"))
 (segment (start 48.6 92.366) (end 45.276 92.366) (width 0.4) (layer "F.Cu") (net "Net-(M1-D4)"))
 (segment (start 74.276 42.306) (end 74.276 92.366) (width 0.4) (layer "F.Cu") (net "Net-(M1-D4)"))
 (segment (start 71.54 93.366) (end 49.6 93.366) (width 0.4) (layer "F.Cu") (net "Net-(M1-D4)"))
 (segment (start 79.661 41.306) (end 75.276 41.306) (width 0.4) (layer "F.Cu") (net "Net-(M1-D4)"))
 (segment (start 49.6 93.366) (end 48.6 92.366) (width 0.4) (layer "F.Cu") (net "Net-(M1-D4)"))
 (segment (start 73.276 79.966) (end 72.276 80.966) (width 0.4) (layer "F.Cu") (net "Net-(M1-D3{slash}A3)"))
 (segment (start 79.661 38.766) (end 74.276 38.766) (width 0.4) (layer "F.Cu") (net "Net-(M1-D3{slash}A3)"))
 (segment (start 74.276 38.766) (end 73.276 39.766) (width 0.4) (layer "F.Cu") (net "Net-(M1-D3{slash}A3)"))
 (segment (start 71.54 80.966) (end 49.6 80.966) (width 0.4) (layer "F.Cu") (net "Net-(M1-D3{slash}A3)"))
 (segment (start 71.54 77.966) (end 71.54 80.966) (width 0.4) (layer "F.Cu") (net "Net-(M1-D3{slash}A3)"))
 (segment (start 72.276 80.966) (end 71.54 80.966) (width 0.4) (layer "F.Cu") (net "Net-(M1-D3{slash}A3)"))
 (segment (start 73.276 39.766) (end 73.276 79.966) (width 0.4) (layer "F.Cu") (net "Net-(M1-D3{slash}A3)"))
 (segment (start 48.6 79.966) (end 45.276 79.966) (width 0.4) (layer "F.Cu") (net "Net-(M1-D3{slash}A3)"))
 (segment (start 49.6 80.966) (end 48.6 79.966) (width 0.4) (layer "F.Cu") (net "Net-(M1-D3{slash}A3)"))
 (segment (start 45.276 65.566) (end 50.575999 65.566) (width 0.4) (layer "F.Cu") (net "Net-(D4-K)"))
 (segment (start 71.276 68.566) (end 49.6 68.566) (width 0.4) (layer "F.Cu") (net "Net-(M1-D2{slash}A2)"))
 (segment (start 72.276 37.226) (end 72.276 67.566) (width 0.4) (layer "F.Cu") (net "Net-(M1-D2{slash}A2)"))
 (segment (start 79.661 36.226) (end 73.276 36.226) (width 0.4) (layer "F.Cu") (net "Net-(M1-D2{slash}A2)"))
 (segment (start 48.6 67.566) (end 45.276 67.566) (width 0.4) (layer "F.Cu") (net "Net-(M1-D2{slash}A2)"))
 (segment (start 72.276 67.566) (end 71.276 68.566) (width 0.4) (layer "F.Cu") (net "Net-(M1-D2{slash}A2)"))
 (segment (start 73.276 36.226) (end 72.276 37.226) (width 0.4) (layer "F.Cu") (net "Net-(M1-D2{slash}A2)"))
 (segment (start 49.6 68.566) (end 48.6 67.566) (width 0.4) (layer "F.Cu") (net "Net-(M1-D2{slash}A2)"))
 (segment (start 53.976 106.666) (end 56.92 106.666) (width 0.4) (layer "F.Cu") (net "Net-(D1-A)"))
 (segment (start 53.976 51.166) (end 56.92 51.166) (width 0.4) (layer "F.Cu") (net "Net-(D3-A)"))
 (segment (start 53.976 65.566) (end 56.92 65.566) (width 0.4) (layer "F.Cu") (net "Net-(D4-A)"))
 (segment (start 45.276 36.766) (end 50.575999 36.766) (width 0.4) (layer "F.Cu") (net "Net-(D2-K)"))
 (segment (start 53.976 36.766) (end 56.92 36.766) (width 0.4) (layer "F.Cu") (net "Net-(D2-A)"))
 (segment (start 53.976 90.366) (end 56.92 90.366) (width 0.4) (layer "F.Cu") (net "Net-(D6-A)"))
 (segment (start 45.276 32.766) (end 48.6 32.766) (width 0.4) (layer "F.Cu") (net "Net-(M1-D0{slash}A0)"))
 (segment (start 50.22 31.146) (end 79.661 31.146) (width 0.4) (layer "F.Cu") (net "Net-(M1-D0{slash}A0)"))
 (segment (start 48.6 32.766) (end 50.22 31.146) (width 0.4) (layer "F.Cu") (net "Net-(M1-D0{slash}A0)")))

